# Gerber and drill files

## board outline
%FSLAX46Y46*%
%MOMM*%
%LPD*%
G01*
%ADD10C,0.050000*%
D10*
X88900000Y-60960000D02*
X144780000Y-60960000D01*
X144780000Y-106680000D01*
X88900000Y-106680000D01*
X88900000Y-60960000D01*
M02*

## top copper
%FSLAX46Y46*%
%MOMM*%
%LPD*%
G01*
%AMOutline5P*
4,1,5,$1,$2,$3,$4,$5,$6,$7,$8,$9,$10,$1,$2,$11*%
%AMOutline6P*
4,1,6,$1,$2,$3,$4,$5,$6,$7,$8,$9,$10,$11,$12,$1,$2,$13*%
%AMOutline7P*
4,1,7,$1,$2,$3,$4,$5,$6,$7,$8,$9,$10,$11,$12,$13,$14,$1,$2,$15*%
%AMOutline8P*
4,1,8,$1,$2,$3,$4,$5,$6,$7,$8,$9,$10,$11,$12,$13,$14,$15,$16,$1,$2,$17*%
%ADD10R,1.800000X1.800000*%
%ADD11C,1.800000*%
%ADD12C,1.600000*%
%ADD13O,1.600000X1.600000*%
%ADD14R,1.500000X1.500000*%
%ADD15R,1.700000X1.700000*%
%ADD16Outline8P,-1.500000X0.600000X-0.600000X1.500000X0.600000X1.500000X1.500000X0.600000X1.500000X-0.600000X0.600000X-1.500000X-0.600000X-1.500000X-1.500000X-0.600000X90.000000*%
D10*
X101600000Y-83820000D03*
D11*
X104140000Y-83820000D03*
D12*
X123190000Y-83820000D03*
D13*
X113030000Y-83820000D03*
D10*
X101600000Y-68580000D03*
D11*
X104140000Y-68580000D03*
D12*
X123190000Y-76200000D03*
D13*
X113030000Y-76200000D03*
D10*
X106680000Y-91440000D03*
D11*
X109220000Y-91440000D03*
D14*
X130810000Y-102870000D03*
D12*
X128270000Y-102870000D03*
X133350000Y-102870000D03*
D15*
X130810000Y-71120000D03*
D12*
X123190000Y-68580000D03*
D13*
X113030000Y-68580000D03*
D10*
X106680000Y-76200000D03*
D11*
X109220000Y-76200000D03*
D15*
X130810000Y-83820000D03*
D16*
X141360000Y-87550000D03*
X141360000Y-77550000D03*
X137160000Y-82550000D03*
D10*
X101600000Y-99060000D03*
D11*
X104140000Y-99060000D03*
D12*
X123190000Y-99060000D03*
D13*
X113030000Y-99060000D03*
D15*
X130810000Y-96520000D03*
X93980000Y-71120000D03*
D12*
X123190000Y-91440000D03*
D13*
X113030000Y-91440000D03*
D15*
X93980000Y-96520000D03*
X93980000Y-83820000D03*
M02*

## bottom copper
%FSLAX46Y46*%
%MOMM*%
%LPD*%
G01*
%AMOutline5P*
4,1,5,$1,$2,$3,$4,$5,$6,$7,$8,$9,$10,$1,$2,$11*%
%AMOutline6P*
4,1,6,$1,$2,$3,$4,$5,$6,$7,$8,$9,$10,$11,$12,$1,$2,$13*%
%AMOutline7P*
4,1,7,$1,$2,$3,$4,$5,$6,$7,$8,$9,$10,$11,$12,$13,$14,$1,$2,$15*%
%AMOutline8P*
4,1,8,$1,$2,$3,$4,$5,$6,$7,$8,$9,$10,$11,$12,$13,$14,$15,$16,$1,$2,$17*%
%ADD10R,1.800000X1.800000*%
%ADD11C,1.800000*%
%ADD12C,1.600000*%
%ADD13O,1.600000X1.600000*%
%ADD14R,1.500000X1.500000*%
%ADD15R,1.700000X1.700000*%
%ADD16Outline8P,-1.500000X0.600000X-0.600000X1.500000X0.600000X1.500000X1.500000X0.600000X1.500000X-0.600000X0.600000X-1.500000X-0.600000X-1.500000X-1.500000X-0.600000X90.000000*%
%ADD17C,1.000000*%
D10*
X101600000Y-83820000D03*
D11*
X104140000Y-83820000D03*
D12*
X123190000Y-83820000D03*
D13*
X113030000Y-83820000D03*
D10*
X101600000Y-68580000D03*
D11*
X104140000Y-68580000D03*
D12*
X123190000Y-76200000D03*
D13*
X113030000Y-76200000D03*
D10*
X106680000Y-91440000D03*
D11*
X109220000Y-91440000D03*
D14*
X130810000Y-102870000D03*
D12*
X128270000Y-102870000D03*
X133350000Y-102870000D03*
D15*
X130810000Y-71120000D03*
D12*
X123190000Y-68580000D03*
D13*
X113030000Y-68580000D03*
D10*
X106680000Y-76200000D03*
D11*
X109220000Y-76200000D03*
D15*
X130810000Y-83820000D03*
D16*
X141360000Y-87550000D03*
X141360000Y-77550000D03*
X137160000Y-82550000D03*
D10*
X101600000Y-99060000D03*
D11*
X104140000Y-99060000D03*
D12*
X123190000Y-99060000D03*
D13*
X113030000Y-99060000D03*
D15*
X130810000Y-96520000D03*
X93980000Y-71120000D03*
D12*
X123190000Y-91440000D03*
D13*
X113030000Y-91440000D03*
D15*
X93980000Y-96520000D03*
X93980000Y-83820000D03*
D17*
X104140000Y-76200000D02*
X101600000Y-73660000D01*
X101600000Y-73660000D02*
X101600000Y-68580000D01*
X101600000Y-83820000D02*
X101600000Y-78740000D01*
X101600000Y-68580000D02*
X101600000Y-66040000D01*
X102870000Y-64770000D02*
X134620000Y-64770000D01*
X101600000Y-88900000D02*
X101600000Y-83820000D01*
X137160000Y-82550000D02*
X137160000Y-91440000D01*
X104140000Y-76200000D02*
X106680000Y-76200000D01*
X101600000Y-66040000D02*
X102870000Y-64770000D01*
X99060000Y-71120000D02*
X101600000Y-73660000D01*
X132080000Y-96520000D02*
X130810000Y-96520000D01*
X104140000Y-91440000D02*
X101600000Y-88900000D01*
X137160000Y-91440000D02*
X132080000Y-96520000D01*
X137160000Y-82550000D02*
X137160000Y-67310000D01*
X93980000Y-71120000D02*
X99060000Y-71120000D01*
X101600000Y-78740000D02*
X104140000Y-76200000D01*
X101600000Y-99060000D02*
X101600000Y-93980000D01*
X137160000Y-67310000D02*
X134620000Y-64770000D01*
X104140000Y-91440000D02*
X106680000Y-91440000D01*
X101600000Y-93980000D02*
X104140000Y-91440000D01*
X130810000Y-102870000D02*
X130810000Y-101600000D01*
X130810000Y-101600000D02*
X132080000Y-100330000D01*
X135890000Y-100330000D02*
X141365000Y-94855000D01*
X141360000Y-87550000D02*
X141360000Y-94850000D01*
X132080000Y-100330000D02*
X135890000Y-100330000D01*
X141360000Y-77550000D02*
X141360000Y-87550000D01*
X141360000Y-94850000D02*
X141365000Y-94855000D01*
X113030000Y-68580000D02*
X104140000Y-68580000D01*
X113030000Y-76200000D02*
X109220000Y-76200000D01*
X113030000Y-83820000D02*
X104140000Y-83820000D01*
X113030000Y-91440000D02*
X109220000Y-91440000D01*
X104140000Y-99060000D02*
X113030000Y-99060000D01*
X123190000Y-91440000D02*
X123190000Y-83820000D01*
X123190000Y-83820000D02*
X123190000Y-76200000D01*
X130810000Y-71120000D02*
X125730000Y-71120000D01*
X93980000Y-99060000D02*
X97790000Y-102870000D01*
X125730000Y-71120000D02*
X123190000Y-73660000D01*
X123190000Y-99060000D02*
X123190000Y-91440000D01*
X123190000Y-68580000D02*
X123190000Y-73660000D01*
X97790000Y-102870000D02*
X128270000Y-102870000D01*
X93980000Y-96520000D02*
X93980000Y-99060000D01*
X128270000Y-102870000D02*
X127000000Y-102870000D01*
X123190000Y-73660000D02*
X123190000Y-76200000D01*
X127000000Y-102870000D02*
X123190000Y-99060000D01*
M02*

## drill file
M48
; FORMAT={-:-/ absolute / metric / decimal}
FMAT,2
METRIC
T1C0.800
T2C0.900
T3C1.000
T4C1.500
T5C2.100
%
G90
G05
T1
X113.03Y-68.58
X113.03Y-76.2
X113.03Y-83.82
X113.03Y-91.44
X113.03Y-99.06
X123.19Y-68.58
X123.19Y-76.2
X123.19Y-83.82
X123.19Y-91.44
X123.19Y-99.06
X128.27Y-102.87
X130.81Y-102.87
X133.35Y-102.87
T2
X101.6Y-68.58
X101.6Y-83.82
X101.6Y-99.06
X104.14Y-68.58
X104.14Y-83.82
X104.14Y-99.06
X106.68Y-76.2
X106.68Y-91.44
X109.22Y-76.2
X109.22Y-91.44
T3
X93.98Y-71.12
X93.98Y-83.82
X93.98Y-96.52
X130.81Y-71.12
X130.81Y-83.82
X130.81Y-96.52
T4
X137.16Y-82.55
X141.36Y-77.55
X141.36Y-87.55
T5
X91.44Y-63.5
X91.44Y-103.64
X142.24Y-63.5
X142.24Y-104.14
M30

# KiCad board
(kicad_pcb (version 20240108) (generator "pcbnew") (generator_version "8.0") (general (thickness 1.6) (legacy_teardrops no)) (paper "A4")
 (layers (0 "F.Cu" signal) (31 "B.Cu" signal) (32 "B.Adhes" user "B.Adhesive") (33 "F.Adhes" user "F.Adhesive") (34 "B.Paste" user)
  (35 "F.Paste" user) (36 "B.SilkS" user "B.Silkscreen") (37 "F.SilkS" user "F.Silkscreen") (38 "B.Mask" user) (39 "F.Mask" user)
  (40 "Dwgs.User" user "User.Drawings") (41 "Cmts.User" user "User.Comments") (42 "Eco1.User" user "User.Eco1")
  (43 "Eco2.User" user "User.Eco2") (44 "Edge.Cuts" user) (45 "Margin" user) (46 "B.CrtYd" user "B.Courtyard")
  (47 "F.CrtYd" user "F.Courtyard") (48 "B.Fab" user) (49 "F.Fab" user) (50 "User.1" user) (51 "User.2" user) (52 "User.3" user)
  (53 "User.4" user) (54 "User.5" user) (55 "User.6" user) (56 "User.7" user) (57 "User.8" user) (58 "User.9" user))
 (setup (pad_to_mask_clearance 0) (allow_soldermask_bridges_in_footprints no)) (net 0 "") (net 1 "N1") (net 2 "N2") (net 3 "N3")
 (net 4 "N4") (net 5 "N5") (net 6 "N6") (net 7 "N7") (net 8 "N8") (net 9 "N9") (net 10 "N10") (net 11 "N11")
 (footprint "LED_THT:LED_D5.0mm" (layer "F.Cu") (at 101.6 83.82)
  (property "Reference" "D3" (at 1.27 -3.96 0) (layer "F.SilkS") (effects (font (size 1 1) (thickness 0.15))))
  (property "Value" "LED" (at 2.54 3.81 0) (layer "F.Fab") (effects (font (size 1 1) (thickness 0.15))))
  (pad "1" thru_hole rect (at 0 0) (size 1.8 1.8) (drill 0.9) (layers "*.Cu" "*.Mask") (remove_unused_layers no) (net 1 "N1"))
  (pad "2" thru_hole circle (at 2.54 0) (size 1.8 1.8) (drill 0.9) (layers "*.Cu" "*.Mask") (remove_unused_layers no) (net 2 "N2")))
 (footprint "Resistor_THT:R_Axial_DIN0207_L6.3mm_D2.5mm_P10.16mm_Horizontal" (layer "F.Cu") (at 123.19 83.82 180)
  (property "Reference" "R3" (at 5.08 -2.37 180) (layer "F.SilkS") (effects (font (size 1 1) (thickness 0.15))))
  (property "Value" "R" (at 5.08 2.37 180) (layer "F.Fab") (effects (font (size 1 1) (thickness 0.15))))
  (pad "1" thru_hole circle (at 0 0 180) (size 1.6 1.6) (drill 0.8) (layers "*.Cu" "*.Mask") (remove_unused_layers no) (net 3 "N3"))
  (pad "2" thru_hole oval (at 10.16 0 180) (size 1.6 1.6) (drill 0.8) (layers "*.Cu" "*.Mask") (remove_unused_layers no) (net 2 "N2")))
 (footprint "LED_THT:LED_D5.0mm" (layer "F.Cu") (at 101.6 68.58)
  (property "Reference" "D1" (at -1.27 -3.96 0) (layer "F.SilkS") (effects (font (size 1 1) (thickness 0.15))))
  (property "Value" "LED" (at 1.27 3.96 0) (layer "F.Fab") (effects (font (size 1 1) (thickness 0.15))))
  (pad "1" thru_hole rect (at 0 0) (size 1.8 1.8) (drill 0.9) (layers "*.Cu" "*.Mask") (remove_unused_layers no) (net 1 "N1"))
  (pad "2" thru_hole circle (at 2.54 0) (size 1.8 1.8) (drill 0.9) (layers "*.Cu" "*.Mask") (remove_unused_layers no) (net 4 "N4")))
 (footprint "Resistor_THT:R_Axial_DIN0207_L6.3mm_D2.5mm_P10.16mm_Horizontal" (layer "F.Cu") (at 123.19 76.2 180)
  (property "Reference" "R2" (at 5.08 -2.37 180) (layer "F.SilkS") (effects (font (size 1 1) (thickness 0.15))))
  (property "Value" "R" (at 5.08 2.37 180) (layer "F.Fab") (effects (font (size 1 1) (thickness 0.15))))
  (pad "1" thru_hole circle (at 0 0 180) (size 1.6 1.6) (drill 0.8) (layers "*.Cu" "*.Mask") (remove_unused_layers no) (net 3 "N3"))
  (pad "2" thru_hole oval (at 10.16 0 180) (size 1.6 1.6) (drill 0.8) (layers "*.Cu" "*.Mask") (remove_unused_layers no) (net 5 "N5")))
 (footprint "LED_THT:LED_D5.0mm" (layer "F.Cu") (at 106.68 91.44)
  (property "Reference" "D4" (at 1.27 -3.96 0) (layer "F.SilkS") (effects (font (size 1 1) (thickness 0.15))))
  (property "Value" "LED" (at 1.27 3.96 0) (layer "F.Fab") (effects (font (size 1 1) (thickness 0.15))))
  (pad "1" thru_hole rect (at 0 0) (size 1.8 1.8) (drill 0.9) (layers "*.Cu" "*.Mask") (remove_unused_layers no) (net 1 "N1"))
  (pad "2" thru_hole circle (at 2.54 0) (size 1.8 1.8) (drill 0.9) (layers "*.Cu" "*.Mask") (remove_unused_layers no) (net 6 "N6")))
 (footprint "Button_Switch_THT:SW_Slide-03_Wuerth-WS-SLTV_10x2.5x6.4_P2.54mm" (layer "F.Cu") (at 130.81 102.87)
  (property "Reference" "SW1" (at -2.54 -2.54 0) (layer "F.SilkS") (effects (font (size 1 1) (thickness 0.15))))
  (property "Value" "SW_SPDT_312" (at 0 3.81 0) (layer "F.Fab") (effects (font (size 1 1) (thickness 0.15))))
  (pad "1" thru_hole rect (at 0 0) (size 1.5 1.5) (drill 0.8) (layers "*.Cu" "*.Mask") (remove_unused_layers no) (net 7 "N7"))
  (pad "2" thru_hole circle (at -2.54 0) (size 1.6 1.6) (drill 0.8) (layers "*.Cu" "*.Mask") (remove_unused_layers no) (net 3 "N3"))
  (pad "3" thru_hole circle (at 2.54 0) (size 1.6 1.6) (drill 0.8) (layers "*.Cu" "*.Mask") (remove_unused_layers no) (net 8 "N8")))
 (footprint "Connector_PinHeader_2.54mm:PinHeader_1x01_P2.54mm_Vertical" (layer "F.Cu") (at 130.81 71.12)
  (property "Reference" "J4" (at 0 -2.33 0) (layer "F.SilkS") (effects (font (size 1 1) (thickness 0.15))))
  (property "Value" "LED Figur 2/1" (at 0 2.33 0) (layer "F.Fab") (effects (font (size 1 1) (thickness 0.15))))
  (pad "1" thru_hole rect (at 0 0) (size 1.7 1.7) (drill 1) (layers "*.Cu" "*.Mask") (remove_unused_layers no) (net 3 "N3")))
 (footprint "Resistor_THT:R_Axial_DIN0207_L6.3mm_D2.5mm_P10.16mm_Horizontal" (layer "F.Cu") (at 123.19 68.58 180)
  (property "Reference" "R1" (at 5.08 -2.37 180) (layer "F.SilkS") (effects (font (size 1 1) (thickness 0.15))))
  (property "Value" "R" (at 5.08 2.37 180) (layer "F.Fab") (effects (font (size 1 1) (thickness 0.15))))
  (pad "1" thru_hole circle (at 0 0 180) (size 1.6 1.6) (drill 0.8) (layers "*.Cu" "*.Mask") (remove_unused_layers no) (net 3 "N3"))
  (pad "2" thru_hole oval (at 10.16 0 180) (size 1.6 1.6) (drill 0.8) (layers "*.Cu" "*.Mask") (remove_unused_layers no) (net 4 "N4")))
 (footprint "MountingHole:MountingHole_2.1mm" (layer "F.Cu") (at 91.44 63.5)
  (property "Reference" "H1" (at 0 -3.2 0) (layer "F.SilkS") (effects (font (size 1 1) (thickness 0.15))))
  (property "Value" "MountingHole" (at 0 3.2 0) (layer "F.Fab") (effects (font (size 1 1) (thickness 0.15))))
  (pad "" np_thru_hole circle (at 0 0) (size 2.1 2.1) (drill 2.1) (layers "*.Cu" "*.Mask")))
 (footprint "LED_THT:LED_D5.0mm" (layer "F.Cu") (at 106.68 76.2)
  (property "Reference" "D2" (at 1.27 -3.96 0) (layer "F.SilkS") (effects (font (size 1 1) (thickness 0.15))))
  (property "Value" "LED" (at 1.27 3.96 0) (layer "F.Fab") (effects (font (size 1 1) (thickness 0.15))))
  (pad "1" thru_hole rect (at 0 0) (size 1.8 1.8) (drill 0.9) (layers "*.Cu" "*.Mask") (remove_unused_layers no) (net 1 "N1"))
  (pad "2" thru_hole circle (at 2.54 0) (size 1.8 1.8) (drill 0.9) (layers "*.Cu" "*.Mask") (remove_unused_layers no) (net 5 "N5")))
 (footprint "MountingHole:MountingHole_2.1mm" (layer "F.Cu") (at 91.44 103.64)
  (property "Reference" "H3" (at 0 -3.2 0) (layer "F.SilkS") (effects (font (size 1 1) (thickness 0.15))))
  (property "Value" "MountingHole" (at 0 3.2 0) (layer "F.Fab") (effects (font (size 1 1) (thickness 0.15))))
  (pad "" np_thru_hole circle (at 0 0) (size 2.1 2.1) (drill 2.1) (layers "*.Cu" "*.Mask")))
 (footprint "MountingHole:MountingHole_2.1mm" (layer "F.Cu") (at 142.24 104.14)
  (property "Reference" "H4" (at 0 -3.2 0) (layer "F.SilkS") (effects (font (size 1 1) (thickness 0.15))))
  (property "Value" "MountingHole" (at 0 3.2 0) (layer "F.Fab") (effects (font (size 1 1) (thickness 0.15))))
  (pad "" np_thru_hole circle (at 0 0) (size 2.1 2.1) (drill 2.1) (layers "*.Cu" "*.Mask")))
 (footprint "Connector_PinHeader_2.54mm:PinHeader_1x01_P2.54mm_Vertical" (layer "F.Cu") (at 130.81 83.82)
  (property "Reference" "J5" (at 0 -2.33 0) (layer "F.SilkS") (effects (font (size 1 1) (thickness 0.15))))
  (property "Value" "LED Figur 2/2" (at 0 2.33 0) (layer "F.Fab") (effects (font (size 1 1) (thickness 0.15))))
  (pad "1" thru_hole rect (at 0 0) (size 1.7 1.7) (drill 1) (layers "*.Cu" "*.Mask") (remove_unused_layers no) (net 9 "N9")))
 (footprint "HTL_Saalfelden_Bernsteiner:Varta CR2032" (layer "F.Cu") (at 137.16 82.55 90)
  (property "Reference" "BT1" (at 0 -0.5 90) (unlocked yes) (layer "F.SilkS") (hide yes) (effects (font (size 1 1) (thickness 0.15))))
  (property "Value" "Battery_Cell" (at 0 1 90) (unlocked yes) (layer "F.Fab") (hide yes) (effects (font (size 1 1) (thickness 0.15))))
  (pad "1" thru_hole roundrect (at -5 4.2 90) (size 3 3) (drill 1.5) (layers "*.Cu" "*.Mask") (remove_unused_layers no) (roundrect_rratio 0)
   (chamfer_ratio 0.3) (chamfer top_left top_right bottom_left bottom_right) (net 7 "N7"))
  (pad "1" thru_hole roundrect (at 5 4.2 90) (size 3 3) (drill 1.5) (layers "*.Cu" "*.Mask") (remove_unused_layers no) (roundrect_rratio 0)
   (chamfer_ratio 0.3) (chamfer top_left top_right bottom_left bottom_right) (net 7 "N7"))
  (pad "2" thru_hole roundrect (at 0 0 90) (size 3 3) (drill 1.5) (layers "*.Cu" "*.Mask") (remove_unused_layers no) (roundrect_rratio 0)
   (chamfer_ratio 0.3) (chamfer top_left top_right bottom_left bottom_right) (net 1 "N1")))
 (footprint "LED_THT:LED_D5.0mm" (layer "F.Cu") (at 101.6 99.06)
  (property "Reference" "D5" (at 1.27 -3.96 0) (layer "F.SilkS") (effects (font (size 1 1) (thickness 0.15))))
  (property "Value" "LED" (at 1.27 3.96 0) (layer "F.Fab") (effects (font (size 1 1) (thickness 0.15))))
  (pad "1" thru_hole rect (at 0 0) (size 1.8 1.8) (drill 0.9) (layers "*.Cu" "*.Mask") (remove_unused_layers no) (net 1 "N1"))
  (pad "2" thru_hole circle (at 2.54 0) (size 1.8 1.8) (drill 0.9) (layers "*.Cu" "*.Mask") (remove_unused_layers no) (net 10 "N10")))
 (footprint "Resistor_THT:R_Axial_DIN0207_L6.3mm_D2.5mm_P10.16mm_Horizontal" (layer "F.Cu") (at 123.19 99.06 180)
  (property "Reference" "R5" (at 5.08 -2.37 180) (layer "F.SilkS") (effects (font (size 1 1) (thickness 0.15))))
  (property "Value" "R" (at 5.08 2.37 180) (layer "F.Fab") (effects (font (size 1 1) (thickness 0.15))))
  (pad "1" thru_hole circle (at 0 0 180) (size 1.6 1.6) (drill 0.8) (layers "*.Cu" "*.Mask") (remove_unused_layers no) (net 3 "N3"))
  (pad "2" thru_hole oval (at 10.16 0 180) (size 1.6 1.6) (drill 0.8) (layers "*.Cu" "*.Mask") (remove_unused_layers no) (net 10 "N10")))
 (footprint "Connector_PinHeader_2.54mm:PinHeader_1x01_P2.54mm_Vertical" (layer "F.Cu") (at 130.81 96.52)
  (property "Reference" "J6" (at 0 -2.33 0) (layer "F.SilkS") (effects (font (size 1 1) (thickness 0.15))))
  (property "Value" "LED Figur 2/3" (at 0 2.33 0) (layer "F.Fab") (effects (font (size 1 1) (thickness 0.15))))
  (pad "1" thru_hole rect (at 0 0) (size 1.7 1.7) (drill 1) (layers "*.Cu" "*.Mask") (remove_unused_layers no) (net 1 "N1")))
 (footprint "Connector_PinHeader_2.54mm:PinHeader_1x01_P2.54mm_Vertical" (layer "F.Cu") (at 93.98 71.12)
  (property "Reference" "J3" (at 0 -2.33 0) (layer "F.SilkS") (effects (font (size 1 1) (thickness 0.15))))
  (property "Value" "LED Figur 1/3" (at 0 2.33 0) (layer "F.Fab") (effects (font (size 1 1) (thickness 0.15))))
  (pad "1" thru_hole rect (at 0 0) (size 1.7 1.7) (drill 1) (layers "*.Cu" "*.Mask") (remove_unused_layers no) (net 1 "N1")))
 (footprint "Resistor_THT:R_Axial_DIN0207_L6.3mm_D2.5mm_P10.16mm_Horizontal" (layer "F.Cu") (at 123.19 91.44 180)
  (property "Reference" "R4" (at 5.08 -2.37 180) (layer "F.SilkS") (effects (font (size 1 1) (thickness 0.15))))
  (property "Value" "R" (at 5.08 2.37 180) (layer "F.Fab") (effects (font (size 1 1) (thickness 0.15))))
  (pad "1" thru_hole circle (at 0 0 180) (size 1.6 1.6) (drill 0.8) (layers "*.Cu" "*.Mask") (remove_unused_layers no) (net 3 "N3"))
  (pad "2" thru_hole oval (at 10.16 0 180) (size 1.6 1.6) (drill 0.8) (layers "*.Cu" "*.Mask") (remove_unused_layers no) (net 6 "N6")))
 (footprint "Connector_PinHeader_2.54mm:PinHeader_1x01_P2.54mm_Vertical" (layer "F.Cu") (at 93.98 96.52)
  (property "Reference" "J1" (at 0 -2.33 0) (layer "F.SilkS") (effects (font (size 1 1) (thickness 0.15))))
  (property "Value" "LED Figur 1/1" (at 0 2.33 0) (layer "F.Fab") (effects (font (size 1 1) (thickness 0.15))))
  (pad "1" thru_hole rect (at 0 0) (size 1.7 1.7) (drill 1) (layers "*.Cu" "*.Mask") (remove_unused_layers no) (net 3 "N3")))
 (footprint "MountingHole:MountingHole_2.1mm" (layer "F.Cu") (at 142.24 63.5)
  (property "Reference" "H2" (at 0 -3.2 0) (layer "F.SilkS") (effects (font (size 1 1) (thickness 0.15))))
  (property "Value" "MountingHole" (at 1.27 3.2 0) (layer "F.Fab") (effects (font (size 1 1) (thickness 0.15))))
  (pad "" np_thru_hole circle (at 0 0) (size 2.1 2.1) (drill 2.1) (layers "*.Cu" "*.Mask")))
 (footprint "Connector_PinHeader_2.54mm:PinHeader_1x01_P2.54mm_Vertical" (layer "F.Cu") (at 93.98 83.82)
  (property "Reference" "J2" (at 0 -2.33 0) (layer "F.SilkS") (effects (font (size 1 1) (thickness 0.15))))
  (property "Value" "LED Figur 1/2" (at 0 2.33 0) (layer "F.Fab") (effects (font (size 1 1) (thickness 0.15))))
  (pad "1" thru_hole rect (at 0 0) (size 1.7 1.7) (drill 1) (layers "*.Cu" "*.Mask") (remove_unused_layers no) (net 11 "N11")))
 (gr_rect (start 88.9 60.96) (end 144.78 106.68) (stroke (width 0.05) (type default)) (fill none) (layer "Edge.Cuts"))
 (segment (start 104.14 76.2) (end 101.6 73.66) (width 1) (layer "B.Cu") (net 1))
 (segment (start 101.6 73.66) (end 101.6 68.58) (width 1) (layer "B.Cu") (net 1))
 (segment (start 101.6 83.82) (end 101.6 78.74) (width 1) (layer "B.Cu") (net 1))
 (segment (start 101.6 68.58) (end 101.6 66.04) (width 1) (layer "B.Cu") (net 1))
 (segment (start 102.87 64.77) (end 134.62 64.77) (width 1) (layer "B.Cu") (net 1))
 (segment (start 101.6 88.9) (end 101.6 83.82) (width 1) (layer "B.Cu") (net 1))
 (segment (start 137.16 82.55) (end 137.16 91.44) (width 1) (layer "B.Cu") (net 1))
 (segment (start 104.14 76.2) (end 106.68 76.2) (width 1) (layer "B.Cu") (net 1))
 (segment (start 101.6 66.04) (end 102.87 64.77) (width 1) (layer "B.Cu") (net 1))
 (segment (start 99.06 71.12) (end 101.6 73.66) (width 1) (layer "B.Cu") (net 1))
 (segment (start 132.08 96.52) (end 130.81 96.52) (width 1) (layer "B.Cu") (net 1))
 (segment (start 104.14 91.44) (end 101.6 88.9) (width 1) (layer "B.Cu") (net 1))
 (segment (start 137.16 91.44) (end 132.08 96.52) (width 1) (layer "B.Cu") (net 1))
 (segment (start 137.16 82.55) (end 137.16 67.31) (width 1) (layer "B.Cu") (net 1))
 (segment (start 93.98 71.12) (end 99.06 71.12) (width 1) (layer "B.Cu") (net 1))
 (segment (start 101.6 78.74) (end 104.14 76.2) (width 1) (layer "B.Cu") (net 1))
 (segment (start 101.6 99.06) (end 101.6 93.98) (width 1) (layer "B.Cu") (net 1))
 (segment (start 137.16 67.31) (end 134.62 64.77) (width 1) (layer "B.Cu") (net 1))
 (segment (start 104.14 91.44) (end 106.68 91.44) (width 1) (layer "B.Cu") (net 1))
 (segment (start 101.6 93.98) (end 104.14 91.44) (width 1) (layer "B.Cu") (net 1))
 (segment (start 130.81 102.87) (end 130.81 101.6) (width 1) (layer "B.Cu") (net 7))
 (segment (start 130.81 101.6) (end 132.08 100.33) (width 1) (layer "B.Cu") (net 7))
 (segment (start 135.89 100.33) (end 141.365 94.855) (width 1) (layer "B.Cu") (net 7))
 (segment (start 141.36 87.55) (end 141.36 94.85) (width 1) (layer "B.Cu") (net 7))
 (segment (start 132.08 100.33) (end 135.89 100.33) (width 1) (layer "B.Cu") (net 7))
 (segment (start 141.36 77.55) (end 141.36 87.55) (width 1) (layer "B.Cu") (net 7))
 (segment (start 141.36 94.85) (end 141.365 94.855) (width 1) (layer "B.Cu") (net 7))
 (segment (start 113.03 68.58) (end 104.14 68.58) (width 1) (layer "B.Cu") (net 4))
 (segment (start 113.03 76.2) (end 109.22 76.2) (width 1) (layer "B.Cu") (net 5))
 (segment (start 113.03 83.82) (end 104.14 83.82) (width 1) (layer "B.Cu") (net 2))
 (segment (start 113.03 91.44) (end 109.22 91.44) (width 1) (layer "B.Cu") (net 6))
 (segment (start 104.14 99.06) (end 113.03 99.06) (width 1) (layer "B.Cu") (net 10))
 (segment (start 123.19 91.44) (end 123.19 83.82) (width 1) (layer "B.Cu") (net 3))
 (segment (start 123.19 83.82) (end 123.19 76.2) (width 1) (layer "B.Cu") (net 3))
 (segment (start 130.81 71.12) (end 125.73 71.12) (width 1) (layer "B.Cu") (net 3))
 (segment (start 93.98 99.06) (end 97.79 102.87) (width 1) (layer "B.Cu") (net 3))
 (segment (start 125.73 71.12) (end 123.19 73.66) (width 1) (layer "B.Cu") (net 3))
 (segment (start 123.19 99.06) (end 123.19 91.44) (width 1) (layer "B.Cu") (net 3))
 (segment (start 123.19 68.58) (end 123.19 73.66) (width 1) (layer "B.Cu") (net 3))
 (segment (start 97.79 102.87) (end 128.27 102.87) (width 1) (layer "B.Cu") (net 3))
 (segment (start 93.98 96.52) (end 93.98 99.06) (width 1) (layer "B.Cu") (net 3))
 (segment (start 128.27 102.87) (end 127 102.87) (width 1) (layer "B.Cu") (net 3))
 (segment (start 123.19 73.66) (end 123.19 76.2) (width 1) (layer "B.Cu") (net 3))
 (segment (start 127 102.87) (end 123.19 99.06) (width 1) (layer "B.Cu") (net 3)))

